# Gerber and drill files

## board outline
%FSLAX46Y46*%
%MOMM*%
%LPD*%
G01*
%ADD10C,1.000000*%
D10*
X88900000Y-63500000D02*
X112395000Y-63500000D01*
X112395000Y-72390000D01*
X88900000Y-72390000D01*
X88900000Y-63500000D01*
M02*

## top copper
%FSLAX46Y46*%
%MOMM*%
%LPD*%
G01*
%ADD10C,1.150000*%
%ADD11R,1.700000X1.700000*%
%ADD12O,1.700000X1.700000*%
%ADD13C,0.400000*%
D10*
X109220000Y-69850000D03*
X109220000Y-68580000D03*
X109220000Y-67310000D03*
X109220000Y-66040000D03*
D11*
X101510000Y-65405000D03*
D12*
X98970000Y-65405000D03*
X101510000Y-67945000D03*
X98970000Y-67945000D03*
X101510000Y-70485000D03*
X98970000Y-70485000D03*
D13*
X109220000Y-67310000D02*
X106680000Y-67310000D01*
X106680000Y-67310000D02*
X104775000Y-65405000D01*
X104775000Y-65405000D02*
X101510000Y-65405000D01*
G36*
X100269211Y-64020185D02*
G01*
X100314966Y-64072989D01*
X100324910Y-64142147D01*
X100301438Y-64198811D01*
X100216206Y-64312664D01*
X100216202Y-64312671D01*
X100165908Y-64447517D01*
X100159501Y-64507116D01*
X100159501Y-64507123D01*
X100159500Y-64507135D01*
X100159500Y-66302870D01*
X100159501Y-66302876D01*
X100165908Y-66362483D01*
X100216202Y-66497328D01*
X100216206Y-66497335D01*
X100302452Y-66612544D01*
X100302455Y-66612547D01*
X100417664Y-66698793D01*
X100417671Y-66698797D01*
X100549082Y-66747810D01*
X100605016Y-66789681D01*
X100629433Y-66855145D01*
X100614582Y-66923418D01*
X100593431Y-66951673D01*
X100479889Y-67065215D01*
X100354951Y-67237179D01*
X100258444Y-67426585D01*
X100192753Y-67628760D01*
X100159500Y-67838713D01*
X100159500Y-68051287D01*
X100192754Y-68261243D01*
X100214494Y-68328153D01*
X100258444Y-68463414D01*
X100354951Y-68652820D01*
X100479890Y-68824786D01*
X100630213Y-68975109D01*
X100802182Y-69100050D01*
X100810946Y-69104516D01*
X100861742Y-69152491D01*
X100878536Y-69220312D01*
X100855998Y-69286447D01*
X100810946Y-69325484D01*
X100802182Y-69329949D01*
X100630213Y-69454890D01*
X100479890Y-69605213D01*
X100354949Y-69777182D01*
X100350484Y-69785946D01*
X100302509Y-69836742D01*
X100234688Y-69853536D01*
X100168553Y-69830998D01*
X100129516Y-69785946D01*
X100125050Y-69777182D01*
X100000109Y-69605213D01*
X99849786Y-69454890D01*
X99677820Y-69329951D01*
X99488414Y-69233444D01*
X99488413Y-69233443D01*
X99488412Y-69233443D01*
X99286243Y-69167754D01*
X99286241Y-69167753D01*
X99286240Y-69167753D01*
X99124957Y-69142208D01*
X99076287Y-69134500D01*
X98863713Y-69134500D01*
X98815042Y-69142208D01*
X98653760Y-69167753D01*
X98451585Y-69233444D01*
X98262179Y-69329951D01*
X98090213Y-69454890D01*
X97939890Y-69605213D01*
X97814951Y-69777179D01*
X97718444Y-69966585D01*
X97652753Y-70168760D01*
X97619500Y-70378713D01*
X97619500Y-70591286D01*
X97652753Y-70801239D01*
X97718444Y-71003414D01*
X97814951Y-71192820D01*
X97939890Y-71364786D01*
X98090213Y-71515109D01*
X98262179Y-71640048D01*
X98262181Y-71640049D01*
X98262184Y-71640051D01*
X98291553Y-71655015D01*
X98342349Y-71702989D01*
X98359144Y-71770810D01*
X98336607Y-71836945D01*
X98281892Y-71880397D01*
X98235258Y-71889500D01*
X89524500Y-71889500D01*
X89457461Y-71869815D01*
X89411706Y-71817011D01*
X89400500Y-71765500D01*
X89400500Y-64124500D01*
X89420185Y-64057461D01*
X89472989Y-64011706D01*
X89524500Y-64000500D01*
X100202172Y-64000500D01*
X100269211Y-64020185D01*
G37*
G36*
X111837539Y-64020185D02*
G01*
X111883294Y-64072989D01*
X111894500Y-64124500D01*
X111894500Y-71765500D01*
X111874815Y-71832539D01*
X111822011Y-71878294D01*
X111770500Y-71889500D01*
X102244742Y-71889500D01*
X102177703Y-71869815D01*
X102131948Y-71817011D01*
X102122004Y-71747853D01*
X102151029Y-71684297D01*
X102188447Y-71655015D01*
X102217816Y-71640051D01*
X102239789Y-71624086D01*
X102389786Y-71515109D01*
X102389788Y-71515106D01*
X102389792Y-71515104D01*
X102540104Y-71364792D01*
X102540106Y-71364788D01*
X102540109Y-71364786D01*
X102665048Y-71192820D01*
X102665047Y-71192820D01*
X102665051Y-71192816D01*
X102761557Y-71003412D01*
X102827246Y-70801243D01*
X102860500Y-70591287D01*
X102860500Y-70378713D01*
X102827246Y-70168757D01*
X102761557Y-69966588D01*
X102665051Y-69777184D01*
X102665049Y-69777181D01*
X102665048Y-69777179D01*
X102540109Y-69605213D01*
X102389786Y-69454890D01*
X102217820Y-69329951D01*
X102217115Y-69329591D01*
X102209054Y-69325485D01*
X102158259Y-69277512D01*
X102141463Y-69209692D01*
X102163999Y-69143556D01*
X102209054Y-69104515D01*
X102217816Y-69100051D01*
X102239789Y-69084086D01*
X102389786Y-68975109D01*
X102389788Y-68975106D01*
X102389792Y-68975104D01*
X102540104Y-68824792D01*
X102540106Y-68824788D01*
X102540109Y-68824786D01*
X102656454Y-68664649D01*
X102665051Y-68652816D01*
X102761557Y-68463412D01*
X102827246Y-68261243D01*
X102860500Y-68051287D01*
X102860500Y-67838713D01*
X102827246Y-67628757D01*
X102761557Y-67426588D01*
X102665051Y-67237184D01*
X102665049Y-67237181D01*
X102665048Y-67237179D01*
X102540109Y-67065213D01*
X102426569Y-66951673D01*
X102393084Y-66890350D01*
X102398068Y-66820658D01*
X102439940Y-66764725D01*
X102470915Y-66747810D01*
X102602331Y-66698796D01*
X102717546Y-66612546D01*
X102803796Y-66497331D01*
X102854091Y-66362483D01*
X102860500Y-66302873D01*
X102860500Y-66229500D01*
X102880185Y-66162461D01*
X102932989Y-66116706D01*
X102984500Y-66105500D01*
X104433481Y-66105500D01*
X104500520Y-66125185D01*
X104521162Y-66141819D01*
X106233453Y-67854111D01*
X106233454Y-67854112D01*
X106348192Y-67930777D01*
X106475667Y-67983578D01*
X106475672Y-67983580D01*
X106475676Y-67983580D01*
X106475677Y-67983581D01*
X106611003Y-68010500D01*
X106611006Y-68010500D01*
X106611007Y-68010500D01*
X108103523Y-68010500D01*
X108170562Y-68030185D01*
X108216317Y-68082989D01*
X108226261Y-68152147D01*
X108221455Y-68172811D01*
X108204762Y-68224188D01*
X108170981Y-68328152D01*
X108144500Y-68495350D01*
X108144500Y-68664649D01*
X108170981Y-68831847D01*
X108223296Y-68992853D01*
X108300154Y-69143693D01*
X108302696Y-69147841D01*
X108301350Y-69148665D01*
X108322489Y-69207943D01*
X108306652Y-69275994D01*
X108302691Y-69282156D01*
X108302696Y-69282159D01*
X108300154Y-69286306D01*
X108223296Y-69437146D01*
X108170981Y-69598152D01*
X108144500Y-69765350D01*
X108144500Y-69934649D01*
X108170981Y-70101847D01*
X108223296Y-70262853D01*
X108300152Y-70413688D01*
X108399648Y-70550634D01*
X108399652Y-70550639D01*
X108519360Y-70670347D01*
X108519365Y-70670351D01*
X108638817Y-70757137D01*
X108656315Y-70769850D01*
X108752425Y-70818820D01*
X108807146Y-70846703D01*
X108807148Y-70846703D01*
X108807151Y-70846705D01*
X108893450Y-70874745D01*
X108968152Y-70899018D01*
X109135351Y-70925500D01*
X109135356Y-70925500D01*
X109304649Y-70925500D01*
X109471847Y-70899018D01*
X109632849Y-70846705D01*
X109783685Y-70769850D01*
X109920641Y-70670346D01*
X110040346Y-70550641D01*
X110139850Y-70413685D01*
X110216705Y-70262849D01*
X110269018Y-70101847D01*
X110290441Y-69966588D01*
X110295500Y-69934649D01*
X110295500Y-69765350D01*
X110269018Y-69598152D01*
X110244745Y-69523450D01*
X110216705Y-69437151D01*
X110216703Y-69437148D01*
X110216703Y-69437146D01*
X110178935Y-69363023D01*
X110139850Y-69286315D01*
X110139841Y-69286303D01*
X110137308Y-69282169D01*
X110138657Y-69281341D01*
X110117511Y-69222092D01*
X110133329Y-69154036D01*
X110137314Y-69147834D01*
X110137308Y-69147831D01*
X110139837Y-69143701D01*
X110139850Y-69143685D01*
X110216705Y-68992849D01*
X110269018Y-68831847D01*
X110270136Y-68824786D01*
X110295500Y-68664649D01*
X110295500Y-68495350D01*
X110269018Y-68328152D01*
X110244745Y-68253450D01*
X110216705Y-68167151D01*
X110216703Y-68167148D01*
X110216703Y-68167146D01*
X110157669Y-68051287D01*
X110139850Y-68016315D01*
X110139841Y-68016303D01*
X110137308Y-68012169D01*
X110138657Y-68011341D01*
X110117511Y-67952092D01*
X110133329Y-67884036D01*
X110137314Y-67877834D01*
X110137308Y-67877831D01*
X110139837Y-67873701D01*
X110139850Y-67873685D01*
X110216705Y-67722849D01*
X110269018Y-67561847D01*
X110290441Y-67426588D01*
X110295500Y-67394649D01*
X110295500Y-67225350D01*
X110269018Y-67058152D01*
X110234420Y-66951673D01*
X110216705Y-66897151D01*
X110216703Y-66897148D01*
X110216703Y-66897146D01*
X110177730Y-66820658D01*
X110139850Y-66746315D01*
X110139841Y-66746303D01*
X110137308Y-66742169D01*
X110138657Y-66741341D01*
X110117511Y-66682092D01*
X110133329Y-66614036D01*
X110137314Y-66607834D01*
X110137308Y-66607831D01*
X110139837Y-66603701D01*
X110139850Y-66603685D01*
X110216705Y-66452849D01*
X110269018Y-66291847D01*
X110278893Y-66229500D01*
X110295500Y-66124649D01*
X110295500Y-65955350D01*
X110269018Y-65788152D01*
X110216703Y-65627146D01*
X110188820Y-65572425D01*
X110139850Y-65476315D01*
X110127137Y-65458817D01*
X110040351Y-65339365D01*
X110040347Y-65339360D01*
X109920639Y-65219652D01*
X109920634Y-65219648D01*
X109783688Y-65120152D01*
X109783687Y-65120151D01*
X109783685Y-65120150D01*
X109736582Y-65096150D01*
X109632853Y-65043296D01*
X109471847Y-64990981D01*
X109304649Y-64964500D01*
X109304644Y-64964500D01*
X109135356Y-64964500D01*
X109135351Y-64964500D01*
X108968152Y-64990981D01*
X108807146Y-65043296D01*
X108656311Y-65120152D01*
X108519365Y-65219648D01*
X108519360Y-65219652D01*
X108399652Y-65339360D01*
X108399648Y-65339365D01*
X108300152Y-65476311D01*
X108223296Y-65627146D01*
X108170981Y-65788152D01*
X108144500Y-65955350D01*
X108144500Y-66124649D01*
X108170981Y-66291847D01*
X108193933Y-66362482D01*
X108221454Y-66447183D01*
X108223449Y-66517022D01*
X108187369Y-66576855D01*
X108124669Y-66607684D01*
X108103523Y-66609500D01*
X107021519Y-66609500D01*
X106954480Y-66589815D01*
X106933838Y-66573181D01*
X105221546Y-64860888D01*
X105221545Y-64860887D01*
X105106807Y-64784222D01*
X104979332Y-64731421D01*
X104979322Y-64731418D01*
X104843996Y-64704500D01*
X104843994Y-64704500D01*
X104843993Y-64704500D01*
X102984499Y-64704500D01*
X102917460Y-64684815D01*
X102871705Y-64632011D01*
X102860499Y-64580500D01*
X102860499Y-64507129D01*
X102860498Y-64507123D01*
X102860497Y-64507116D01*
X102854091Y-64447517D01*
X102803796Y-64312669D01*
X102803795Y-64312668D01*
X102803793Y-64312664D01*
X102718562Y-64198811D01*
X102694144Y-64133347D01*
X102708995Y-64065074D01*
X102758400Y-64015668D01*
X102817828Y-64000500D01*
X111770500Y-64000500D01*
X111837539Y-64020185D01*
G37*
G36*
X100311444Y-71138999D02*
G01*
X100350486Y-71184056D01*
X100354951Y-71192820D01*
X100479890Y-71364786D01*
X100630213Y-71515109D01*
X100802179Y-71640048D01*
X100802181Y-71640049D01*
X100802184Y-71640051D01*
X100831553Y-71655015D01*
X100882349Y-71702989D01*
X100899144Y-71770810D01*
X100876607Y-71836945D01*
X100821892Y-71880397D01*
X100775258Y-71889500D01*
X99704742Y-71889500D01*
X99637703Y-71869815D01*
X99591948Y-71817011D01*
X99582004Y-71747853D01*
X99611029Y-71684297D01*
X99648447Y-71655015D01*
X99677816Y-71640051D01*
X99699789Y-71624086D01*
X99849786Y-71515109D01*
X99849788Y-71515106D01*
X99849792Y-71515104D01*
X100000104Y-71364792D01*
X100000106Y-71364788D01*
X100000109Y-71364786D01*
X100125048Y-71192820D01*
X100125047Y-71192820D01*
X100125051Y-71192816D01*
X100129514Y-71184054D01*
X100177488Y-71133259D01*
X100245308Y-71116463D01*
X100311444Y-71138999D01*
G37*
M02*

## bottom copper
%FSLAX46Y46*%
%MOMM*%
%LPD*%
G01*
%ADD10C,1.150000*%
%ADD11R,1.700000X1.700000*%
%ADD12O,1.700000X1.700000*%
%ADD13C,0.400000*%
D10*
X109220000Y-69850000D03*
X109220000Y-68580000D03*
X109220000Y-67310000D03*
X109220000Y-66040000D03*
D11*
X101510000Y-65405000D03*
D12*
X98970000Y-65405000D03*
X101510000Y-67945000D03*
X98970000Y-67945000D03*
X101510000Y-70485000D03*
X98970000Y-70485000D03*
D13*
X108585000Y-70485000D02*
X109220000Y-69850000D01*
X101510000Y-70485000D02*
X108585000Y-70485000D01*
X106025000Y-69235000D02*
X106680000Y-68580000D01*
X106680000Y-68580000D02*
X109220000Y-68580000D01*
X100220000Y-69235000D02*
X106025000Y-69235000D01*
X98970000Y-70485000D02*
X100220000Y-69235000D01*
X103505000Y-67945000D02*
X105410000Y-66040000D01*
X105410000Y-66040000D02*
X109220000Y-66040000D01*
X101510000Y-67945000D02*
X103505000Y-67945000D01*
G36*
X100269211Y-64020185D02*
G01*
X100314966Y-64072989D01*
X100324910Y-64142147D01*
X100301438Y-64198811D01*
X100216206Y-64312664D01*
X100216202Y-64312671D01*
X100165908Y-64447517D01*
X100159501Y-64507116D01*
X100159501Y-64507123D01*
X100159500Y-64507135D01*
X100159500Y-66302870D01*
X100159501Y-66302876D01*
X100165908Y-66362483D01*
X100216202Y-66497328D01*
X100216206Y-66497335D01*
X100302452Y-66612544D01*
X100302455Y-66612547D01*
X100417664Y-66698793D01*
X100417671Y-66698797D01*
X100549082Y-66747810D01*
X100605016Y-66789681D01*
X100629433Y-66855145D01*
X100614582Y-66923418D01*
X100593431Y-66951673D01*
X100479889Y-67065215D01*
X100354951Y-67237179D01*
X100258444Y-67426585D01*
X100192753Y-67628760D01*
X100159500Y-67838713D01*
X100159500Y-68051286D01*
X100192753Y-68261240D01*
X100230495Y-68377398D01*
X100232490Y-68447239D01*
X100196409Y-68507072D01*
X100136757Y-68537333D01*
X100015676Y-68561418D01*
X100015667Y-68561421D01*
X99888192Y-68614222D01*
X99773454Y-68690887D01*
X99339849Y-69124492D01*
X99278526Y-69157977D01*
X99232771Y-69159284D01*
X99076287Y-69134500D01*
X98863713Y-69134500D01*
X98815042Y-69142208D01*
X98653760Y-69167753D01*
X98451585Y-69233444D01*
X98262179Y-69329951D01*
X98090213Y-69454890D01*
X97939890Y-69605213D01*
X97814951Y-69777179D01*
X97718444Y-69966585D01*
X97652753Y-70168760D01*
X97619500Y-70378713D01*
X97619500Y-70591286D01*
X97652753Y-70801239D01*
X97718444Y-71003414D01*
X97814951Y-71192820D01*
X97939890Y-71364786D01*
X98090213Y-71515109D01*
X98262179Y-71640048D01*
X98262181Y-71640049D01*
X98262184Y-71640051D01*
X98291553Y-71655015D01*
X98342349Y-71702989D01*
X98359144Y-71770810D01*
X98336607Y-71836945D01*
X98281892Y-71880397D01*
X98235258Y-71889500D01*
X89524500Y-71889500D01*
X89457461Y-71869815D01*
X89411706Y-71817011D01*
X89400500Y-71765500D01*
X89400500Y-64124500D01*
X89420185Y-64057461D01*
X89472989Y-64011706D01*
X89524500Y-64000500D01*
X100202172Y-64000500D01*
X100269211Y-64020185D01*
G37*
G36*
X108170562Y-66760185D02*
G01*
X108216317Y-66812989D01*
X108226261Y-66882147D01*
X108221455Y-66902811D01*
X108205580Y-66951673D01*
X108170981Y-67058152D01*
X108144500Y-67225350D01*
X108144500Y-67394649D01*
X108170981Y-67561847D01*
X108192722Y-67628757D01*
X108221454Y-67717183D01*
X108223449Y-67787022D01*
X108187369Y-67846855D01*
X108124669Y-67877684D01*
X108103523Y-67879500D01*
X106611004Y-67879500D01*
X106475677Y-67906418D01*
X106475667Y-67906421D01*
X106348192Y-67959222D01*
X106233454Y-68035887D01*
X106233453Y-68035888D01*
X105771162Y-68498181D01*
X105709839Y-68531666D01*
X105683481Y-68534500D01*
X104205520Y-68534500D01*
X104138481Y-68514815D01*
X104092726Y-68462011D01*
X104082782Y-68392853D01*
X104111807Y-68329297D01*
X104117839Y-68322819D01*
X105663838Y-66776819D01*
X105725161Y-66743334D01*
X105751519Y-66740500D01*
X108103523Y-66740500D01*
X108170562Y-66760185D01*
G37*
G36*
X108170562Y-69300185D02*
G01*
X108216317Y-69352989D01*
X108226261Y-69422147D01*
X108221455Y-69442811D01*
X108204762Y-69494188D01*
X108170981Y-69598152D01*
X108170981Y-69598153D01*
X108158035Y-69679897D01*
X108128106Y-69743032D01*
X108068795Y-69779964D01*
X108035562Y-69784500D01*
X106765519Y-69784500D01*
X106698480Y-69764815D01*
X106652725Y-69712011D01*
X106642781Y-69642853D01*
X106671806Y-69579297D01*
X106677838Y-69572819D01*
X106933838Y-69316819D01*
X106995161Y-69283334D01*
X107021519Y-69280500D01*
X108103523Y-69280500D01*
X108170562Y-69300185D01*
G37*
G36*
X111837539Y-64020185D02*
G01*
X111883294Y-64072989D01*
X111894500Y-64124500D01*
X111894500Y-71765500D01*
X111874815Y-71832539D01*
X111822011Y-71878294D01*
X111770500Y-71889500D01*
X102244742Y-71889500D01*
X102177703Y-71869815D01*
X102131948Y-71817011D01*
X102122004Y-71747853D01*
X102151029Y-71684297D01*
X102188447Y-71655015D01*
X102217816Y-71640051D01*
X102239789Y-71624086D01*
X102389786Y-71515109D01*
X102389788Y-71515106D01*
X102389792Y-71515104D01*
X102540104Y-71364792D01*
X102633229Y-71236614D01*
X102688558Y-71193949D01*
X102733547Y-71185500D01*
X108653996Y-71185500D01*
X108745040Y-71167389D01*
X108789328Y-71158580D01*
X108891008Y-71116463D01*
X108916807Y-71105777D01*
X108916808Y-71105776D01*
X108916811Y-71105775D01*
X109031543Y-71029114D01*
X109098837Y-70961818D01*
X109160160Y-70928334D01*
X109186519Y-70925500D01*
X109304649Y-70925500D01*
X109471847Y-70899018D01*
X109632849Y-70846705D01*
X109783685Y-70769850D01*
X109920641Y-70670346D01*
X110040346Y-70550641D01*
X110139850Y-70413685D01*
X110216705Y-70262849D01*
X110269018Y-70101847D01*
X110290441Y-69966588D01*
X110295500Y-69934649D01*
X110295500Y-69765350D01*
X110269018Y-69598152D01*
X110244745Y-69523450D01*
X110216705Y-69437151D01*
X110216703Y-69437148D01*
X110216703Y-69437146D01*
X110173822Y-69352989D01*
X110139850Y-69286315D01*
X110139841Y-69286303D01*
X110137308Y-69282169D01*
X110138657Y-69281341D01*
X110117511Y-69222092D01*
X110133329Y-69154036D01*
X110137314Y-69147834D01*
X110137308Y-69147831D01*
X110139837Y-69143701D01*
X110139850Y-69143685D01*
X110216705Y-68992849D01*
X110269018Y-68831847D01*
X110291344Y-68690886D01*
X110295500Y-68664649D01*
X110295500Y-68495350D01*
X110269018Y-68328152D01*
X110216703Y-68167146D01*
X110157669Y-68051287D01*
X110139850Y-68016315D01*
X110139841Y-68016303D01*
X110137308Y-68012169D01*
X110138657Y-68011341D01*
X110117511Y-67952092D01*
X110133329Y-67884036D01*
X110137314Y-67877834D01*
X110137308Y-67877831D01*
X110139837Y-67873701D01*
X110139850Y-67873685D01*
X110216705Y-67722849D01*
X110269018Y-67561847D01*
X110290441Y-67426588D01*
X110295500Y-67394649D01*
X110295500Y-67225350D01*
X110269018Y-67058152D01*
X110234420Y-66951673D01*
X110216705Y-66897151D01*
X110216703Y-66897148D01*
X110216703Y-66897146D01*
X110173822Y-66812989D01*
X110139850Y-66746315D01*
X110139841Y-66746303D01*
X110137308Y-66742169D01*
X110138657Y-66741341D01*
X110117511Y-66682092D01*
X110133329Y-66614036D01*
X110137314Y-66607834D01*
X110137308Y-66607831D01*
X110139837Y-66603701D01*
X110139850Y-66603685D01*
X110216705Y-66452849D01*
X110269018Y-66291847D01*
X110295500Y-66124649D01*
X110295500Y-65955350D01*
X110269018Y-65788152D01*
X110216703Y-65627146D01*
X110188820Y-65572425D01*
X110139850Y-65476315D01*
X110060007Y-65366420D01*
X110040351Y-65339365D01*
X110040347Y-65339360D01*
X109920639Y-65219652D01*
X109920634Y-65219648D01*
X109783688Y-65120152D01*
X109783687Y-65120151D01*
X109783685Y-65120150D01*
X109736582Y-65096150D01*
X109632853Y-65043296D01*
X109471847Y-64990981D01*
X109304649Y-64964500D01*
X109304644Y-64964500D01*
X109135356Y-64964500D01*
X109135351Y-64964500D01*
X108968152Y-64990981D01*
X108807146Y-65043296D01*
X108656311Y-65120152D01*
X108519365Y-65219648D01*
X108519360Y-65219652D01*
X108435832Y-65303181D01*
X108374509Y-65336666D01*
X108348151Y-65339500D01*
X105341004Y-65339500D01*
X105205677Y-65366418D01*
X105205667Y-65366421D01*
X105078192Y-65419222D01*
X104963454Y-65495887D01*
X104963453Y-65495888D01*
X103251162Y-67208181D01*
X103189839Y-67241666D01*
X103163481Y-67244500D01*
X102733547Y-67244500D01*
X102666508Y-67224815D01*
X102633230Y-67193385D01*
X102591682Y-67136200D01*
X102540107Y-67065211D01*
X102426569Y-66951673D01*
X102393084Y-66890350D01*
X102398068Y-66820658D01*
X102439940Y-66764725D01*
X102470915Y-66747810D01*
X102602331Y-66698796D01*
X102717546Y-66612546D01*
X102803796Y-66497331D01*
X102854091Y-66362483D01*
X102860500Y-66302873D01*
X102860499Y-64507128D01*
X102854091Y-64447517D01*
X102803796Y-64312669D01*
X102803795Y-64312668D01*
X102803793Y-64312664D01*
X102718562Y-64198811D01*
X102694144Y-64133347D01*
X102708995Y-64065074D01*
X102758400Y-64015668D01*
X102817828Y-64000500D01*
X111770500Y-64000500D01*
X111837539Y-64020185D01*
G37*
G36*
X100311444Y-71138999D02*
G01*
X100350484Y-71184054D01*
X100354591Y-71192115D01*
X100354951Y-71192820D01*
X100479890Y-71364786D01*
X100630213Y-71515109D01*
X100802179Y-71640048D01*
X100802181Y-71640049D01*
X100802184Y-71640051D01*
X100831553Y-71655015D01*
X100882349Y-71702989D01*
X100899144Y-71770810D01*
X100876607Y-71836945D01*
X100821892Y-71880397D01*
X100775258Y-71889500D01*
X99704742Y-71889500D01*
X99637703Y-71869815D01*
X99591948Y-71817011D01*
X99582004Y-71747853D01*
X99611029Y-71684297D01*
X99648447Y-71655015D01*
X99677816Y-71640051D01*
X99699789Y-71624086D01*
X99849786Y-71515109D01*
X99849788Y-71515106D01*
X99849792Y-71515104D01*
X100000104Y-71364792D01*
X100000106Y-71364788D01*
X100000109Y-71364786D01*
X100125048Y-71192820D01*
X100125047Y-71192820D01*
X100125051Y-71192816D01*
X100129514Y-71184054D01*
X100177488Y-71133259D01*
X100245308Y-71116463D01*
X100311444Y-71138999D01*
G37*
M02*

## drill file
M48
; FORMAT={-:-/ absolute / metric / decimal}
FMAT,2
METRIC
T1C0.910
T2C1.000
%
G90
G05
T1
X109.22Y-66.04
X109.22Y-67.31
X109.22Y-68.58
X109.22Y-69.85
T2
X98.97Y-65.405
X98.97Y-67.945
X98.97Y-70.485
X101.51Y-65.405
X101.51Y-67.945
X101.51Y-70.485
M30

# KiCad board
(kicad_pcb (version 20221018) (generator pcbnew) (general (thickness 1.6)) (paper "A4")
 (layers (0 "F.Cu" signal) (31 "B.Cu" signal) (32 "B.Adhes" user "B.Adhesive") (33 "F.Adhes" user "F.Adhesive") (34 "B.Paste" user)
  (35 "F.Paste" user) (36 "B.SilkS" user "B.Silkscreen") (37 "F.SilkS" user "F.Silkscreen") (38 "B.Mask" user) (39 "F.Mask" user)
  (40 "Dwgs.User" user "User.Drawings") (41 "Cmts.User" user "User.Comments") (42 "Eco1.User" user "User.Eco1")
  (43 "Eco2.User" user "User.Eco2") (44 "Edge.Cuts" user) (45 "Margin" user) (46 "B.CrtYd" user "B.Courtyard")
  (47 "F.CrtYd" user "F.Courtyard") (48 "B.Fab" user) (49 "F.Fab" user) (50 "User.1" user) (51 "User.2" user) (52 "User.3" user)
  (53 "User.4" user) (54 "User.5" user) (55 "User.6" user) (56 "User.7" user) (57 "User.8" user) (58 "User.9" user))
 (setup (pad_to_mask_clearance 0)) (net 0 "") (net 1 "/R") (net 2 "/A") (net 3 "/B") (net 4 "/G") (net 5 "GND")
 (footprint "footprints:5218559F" (layer "F.Cu") (at 109.22 69.85 180)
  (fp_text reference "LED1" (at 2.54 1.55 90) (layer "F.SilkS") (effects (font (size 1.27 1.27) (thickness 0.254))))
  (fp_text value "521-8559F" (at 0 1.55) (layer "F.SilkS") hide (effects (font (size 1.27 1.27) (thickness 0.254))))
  (pad "1" thru_hole circle (at 0 0 180) (size 1.15 1.15) (drill 0.91) (layers "*.Cu" "*.Mask") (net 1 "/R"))
  (pad "2" thru_hole circle (at 0 1.27 180) (size 1.15 1.15) (drill 0.91) (layers "*.Cu" "*.Mask") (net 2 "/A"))
  (pad "3" thru_hole circle (at 0 2.54 180) (size 1.15 1.15) (drill 0.91) (layers "*.Cu" "*.Mask") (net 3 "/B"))
  (pad "4" thru_hole circle (at 0 3.81 180) (size 1.15 1.15) (drill 0.91) (layers "*.Cu" "*.Mask") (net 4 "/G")))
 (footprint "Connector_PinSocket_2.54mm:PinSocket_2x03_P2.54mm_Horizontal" (layer "F.Cu") (at 101.51 65.405)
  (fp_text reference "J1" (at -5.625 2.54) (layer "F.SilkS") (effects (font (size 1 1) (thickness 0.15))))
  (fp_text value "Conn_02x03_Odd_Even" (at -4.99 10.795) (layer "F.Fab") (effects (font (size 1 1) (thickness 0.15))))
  (pad "1" thru_hole rect (at 0 0) (size 1.7 1.7) (drill 1) (layers "*.Cu" "*.Mask") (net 3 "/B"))
  (pad "2" thru_hole oval (at -2.54 0) (size 1.7 1.7) (drill 1) (layers "*.Cu" "*.Mask") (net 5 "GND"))
  (pad "3" thru_hole oval (at 0 2.54) (size 1.7 1.7) (drill 1) (layers "*.Cu" "*.Mask") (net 4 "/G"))
  (pad "4" thru_hole oval (at -2.54 2.54) (size 1.7 1.7) (drill 1) (layers "*.Cu" "*.Mask") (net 5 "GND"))
  (pad "5" thru_hole oval (at 0 5.08) (size 1.7 1.7) (drill 1) (layers "*.Cu" "*.Mask") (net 1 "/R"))
  (pad "6" thru_hole oval (at -2.54 5.08) (size 1.7 1.7) (drill 1) (layers "*.Cu" "*.Mask") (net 2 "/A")))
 (gr_rect (start 88.9 63.5) (end 112.395 72.39) (stroke (width 1) (type default)) (fill none) (layer "Edge.Cuts"))
 (segment (start 108.585 70.485) (end 109.22 69.85) (width 0.4) (layer "B.Cu") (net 1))
 (segment (start 101.51 70.485) (end 108.585 70.485) (width 0.4) (layer "B.Cu") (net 1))
 (segment (start 106.025 69.235) (end 106.68 68.58) (width 0.4) (layer "B.Cu") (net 2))
 (segment (start 106.68 68.58) (end 109.22 68.58) (width 0.4) (layer "B.Cu") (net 2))
 (segment (start 100.22 69.235) (end 106.025 69.235) (width 0.4) (layer "B.Cu") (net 2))
 (segment (start 98.97 70.485) (end 100.22 69.235) (width 0.4) (layer "B.Cu") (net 2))
 (segment (start 103.505 67.945) (end 105.41 66.04) (width 0.4) (layer "B.Cu") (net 4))
 (segment (start 105.41 66.04) (end 109.22 66.04) (width 0.4) (layer "B.Cu") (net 4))
 (segment (start 101.51 67.945) (end 103.505 67.945) (width 0.4) (layer "B.Cu") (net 4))
 (segment (start 109.22 67.31) (end 106.68 67.31) (width 0.4) (layer "F.Cu") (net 3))
 (segment (start 106.68 67.31) (end 104.775 65.405) (width 0.4) (layer "F.Cu") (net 3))
 (segment (start 104.775 65.405) (end 101.51 65.405) (width 0.4) (layer "F.Cu") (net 3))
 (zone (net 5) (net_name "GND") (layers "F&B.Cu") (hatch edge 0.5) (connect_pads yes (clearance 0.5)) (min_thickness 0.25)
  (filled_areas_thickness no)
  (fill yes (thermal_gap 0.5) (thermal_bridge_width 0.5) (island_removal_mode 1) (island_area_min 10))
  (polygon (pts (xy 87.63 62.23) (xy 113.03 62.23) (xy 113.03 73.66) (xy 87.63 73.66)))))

